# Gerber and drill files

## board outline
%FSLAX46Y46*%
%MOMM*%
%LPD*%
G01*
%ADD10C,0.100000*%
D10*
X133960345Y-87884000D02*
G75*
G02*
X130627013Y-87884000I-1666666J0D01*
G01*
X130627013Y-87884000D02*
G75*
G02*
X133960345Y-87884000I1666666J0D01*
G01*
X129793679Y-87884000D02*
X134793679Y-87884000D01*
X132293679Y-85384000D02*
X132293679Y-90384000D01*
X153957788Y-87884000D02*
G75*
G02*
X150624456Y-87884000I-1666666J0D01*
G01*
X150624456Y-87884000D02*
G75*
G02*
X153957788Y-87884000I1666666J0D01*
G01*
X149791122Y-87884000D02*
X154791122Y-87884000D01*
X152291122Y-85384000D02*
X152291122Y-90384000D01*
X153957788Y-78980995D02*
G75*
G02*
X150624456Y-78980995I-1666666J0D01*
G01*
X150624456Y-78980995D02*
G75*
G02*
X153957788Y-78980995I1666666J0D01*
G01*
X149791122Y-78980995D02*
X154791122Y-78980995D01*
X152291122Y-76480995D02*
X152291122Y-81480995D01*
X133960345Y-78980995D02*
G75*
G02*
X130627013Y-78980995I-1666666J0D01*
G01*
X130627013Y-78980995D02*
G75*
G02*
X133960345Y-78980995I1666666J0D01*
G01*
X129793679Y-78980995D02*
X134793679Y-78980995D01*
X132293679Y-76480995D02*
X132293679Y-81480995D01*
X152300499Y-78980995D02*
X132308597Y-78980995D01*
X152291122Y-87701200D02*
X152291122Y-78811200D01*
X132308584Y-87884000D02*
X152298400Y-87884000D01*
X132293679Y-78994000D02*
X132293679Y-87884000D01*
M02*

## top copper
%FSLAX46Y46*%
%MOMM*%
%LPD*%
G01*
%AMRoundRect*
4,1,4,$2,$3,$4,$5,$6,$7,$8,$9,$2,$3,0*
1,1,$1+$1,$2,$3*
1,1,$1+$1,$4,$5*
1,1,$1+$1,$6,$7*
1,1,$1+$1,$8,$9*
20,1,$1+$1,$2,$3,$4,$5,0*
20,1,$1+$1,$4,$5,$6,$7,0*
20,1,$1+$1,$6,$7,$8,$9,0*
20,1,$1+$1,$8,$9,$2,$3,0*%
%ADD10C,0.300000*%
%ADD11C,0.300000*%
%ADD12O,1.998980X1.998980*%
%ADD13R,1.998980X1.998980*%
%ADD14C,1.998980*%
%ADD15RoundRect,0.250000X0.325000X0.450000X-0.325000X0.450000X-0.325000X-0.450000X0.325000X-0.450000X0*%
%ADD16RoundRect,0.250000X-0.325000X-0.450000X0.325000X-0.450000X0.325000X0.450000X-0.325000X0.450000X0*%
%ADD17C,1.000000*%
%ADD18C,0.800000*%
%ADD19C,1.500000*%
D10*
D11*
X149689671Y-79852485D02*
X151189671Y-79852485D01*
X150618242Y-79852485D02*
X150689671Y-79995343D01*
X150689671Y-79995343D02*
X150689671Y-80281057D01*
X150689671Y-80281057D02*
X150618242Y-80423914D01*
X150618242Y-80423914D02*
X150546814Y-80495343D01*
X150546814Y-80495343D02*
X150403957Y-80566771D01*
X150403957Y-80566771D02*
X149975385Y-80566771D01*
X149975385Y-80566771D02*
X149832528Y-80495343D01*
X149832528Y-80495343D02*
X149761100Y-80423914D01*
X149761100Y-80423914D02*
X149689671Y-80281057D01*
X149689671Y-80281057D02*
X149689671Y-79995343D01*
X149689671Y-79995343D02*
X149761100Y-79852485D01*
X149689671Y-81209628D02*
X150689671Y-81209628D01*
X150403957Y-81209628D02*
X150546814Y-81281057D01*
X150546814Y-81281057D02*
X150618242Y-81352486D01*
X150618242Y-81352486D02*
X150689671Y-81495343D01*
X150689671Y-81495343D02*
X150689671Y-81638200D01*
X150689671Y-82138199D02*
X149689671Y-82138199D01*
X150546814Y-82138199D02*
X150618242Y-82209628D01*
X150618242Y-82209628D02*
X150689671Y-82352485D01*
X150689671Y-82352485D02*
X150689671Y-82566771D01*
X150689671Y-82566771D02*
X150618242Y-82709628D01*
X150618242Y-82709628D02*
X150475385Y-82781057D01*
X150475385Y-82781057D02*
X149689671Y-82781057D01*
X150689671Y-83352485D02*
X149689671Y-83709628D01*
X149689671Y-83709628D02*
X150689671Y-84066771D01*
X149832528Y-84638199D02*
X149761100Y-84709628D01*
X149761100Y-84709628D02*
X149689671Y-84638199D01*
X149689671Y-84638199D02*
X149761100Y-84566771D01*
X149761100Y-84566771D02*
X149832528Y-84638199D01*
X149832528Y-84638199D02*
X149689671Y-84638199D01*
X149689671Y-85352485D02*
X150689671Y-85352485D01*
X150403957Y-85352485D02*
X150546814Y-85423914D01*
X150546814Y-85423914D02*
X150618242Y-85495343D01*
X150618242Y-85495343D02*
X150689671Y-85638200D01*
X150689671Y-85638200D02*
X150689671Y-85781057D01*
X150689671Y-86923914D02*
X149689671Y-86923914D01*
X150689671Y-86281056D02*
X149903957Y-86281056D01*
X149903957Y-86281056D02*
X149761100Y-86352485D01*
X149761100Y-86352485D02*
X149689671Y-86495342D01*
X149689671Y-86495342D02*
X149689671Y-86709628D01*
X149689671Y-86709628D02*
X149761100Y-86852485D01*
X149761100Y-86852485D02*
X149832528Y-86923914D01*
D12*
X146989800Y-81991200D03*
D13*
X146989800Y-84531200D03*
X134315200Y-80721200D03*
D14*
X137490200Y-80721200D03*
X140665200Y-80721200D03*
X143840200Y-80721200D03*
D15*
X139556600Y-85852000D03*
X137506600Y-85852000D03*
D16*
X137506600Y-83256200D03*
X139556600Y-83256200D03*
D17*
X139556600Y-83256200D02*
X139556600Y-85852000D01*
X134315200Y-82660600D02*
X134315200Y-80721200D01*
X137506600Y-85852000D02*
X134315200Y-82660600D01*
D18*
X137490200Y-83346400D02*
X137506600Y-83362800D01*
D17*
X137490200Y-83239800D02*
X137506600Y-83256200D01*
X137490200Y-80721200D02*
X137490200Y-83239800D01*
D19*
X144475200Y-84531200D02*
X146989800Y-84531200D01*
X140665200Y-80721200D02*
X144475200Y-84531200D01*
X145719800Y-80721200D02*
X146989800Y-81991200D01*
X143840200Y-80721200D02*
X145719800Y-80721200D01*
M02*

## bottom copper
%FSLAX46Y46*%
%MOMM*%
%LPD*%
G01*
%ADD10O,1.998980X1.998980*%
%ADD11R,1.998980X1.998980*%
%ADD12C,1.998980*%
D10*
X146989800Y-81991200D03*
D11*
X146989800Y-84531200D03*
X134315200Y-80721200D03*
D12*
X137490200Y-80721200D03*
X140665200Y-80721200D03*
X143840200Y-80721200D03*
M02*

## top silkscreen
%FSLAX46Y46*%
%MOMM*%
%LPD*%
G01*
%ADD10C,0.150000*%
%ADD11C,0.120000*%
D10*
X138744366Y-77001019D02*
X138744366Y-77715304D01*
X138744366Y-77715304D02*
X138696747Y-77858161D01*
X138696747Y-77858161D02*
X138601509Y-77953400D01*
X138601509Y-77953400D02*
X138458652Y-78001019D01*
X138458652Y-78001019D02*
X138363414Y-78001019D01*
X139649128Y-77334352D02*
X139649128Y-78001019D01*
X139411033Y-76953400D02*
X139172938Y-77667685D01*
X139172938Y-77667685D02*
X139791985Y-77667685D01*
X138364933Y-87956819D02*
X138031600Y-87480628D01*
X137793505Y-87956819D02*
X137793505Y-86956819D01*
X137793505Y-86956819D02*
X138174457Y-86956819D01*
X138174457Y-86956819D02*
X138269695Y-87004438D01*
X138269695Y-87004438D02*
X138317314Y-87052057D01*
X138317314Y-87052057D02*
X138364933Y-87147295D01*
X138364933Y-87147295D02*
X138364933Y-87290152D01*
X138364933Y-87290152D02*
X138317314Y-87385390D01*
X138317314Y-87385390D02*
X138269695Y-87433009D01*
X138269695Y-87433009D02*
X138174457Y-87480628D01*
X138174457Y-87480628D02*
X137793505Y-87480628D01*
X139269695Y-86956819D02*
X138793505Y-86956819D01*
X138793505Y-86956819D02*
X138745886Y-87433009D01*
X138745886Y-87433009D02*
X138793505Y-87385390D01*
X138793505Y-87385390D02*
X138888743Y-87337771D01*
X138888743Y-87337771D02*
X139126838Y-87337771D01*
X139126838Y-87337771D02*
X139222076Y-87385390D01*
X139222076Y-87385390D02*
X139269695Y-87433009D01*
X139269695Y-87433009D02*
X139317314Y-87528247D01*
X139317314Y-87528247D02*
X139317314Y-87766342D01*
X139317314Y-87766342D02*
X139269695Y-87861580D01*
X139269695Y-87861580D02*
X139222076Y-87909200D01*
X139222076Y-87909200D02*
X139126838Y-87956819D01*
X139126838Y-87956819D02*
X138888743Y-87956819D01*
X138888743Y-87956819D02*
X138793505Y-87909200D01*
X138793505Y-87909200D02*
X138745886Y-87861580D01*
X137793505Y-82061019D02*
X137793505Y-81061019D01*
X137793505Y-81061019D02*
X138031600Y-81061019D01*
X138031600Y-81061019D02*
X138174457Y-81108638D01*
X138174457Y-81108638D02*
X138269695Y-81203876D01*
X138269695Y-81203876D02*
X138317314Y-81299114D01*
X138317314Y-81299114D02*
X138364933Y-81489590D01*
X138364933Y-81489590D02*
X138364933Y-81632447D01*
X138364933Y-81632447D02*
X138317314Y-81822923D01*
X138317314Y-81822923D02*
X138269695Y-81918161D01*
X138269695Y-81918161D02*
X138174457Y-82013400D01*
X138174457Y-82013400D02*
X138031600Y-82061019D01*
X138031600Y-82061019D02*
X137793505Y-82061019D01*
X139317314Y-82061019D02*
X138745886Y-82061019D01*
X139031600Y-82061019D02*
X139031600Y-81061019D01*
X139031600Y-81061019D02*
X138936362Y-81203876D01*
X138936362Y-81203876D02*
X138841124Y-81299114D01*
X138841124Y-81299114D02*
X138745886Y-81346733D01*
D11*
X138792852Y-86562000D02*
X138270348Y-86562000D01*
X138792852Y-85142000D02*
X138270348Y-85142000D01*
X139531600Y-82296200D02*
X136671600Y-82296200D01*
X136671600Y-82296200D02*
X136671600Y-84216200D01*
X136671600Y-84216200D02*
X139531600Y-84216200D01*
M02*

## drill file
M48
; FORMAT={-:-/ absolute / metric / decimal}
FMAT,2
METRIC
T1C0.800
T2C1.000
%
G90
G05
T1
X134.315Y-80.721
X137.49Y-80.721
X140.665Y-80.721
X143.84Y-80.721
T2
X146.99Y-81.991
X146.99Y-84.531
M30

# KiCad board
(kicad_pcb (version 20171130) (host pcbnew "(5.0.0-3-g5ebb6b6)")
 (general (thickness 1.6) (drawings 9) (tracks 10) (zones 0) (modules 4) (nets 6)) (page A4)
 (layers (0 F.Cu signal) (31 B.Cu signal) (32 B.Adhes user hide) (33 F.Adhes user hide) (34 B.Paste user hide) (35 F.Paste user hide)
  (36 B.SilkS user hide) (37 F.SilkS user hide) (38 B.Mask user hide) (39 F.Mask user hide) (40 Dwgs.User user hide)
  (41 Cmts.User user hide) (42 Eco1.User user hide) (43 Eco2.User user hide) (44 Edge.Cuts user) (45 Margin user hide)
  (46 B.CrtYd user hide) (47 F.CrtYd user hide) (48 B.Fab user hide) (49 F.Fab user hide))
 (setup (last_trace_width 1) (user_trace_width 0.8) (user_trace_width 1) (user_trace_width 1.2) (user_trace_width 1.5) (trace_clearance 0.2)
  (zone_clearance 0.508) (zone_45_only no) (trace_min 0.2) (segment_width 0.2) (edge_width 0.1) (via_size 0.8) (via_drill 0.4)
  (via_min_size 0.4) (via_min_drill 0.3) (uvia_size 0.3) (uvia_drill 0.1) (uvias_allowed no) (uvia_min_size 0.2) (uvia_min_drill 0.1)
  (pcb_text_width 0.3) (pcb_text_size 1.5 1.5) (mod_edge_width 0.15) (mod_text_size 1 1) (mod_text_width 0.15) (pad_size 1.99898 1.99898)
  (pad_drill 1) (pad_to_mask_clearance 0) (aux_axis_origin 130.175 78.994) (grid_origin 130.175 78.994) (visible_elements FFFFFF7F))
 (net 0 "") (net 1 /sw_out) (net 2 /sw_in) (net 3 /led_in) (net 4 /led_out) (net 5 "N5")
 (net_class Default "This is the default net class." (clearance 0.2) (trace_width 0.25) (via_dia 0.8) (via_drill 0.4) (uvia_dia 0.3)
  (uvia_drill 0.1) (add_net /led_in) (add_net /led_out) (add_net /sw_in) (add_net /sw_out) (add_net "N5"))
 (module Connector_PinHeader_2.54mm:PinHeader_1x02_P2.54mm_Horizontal (layer B.Cu) (at 146.9898 84.5312)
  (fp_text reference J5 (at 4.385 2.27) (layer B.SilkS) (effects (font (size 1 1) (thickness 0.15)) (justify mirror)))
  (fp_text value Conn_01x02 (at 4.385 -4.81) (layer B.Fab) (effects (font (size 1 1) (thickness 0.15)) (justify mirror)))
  (pad 2 thru_hole oval (at 0 -2.54) (size 1.99898 1.99898) (drill 1) (layers *.Mask F.Cu) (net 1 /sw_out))
  (pad 1 thru_hole rect (at 0 0) (size 1.99898 1.99898) (drill 1) (layers *.Mask F.Cu) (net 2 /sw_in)))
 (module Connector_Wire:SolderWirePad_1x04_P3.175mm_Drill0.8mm (layer F.Cu) (at 134.3152 80.7212)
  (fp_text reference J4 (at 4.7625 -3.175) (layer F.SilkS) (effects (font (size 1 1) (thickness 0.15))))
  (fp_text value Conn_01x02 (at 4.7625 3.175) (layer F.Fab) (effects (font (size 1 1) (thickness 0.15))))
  (pad 1 thru_hole rect (at 0 0) (size 1.99898 1.99898) (drill 0.8001) (layers *.Cu *.Mask) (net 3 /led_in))
  (pad 2 thru_hole circle (at 3.175 0) (size 1.99898 1.99898) (drill 0.8001) (layers *.Cu *.Mask) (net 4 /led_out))
  (pad 3 thru_hole circle (at 6.35 0) (size 1.99898 1.99898) (drill 0.8001) (layers *.Cu *.Mask) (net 2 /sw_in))
  (pad 4 thru_hole circle (at 9.525 0) (size 1.99898 1.99898) (drill 0.8001) (layers *.Cu *.Mask) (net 1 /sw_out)))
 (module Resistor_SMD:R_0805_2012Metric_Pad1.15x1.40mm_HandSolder (layer F.Cu) (at 138.5316 85.852 180)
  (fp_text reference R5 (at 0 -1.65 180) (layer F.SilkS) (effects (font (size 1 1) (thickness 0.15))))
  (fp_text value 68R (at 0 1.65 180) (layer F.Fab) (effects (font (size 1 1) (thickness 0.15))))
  (fp_line (start -0.261252 -0.71) (end 0.261252 -0.71) (layer F.SilkS) (width 0.12))
  (fp_line (start -0.261252 0.71) (end 0.261252 0.71) (layer F.SilkS) (width 0.12))
  (pad 1 smd roundrect (at -1.025 0 180) (size 1.15 1.4) (layers F.Cu F.Paste F.Mask) (roundrect_rratio 0.217391) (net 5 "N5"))
  (pad 2 smd roundrect (at 1.025 0 180) (size 1.15 1.4) (layers F.Cu F.Paste F.Mask) (roundrect_rratio 0.217391) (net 3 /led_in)))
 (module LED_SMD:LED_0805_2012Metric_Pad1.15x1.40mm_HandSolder (layer F.Cu) (at 138.5316 83.2562)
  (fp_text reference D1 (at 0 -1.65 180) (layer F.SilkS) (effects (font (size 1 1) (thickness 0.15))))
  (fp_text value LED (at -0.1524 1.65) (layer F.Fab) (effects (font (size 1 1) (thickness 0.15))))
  (fp_line (start 1 -0.96) (end -1.86 -0.96) (layer F.SilkS) (width 0.12))
  (fp_line (start -1.86 -0.96) (end -1.86 0.96) (layer F.SilkS) (width 0.12))
  (fp_line (start -1.86 0.96) (end 1 0.96) (layer F.SilkS) (width 0.12))
  (pad 1 smd roundrect (at -1.025 0) (size 1.15 1.4) (layers F.Cu F.Paste F.Mask) (roundrect_rratio 0.217391) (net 4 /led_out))
  (pad 2 smd roundrect (at 1.025 0) (size 1.15 1.4) (layers F.Cu F.Paste F.Mask) (roundrect_rratio 0.217391) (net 5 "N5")))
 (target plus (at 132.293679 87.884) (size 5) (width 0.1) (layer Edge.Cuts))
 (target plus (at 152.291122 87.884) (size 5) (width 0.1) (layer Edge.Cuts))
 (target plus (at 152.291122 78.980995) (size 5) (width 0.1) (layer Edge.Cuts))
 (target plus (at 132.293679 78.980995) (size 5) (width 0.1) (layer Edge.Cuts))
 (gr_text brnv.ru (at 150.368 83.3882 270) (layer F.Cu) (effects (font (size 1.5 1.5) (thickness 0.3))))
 (gr_line (start 152.300499 78.980995) (end 132.308597 78.980995) (layer Edge.Cuts) (width 0.1))
 (gr_line (start 152.291122 87.7012) (end 152.291122 78.8112) (layer Edge.Cuts) (width 0.1))
 (gr_line (start 132.308584 87.884) (end 152.2984 87.884) (layer Edge.Cuts) (width 0.1))
 (gr_line (start 132.293679 78.994) (end 132.293679 87.884) (layer Edge.Cuts) (width 0.1))
 (segment (start 139.5566 83.2562) (end 139.5566 85.852) (width 1) (layer F.Cu) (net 5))
 (segment (start 134.3152 82.6606) (end 134.3152 80.7212) (width 1) (layer F.Cu) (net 3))
 (segment (start 137.5066 85.852) (end 134.3152 82.6606) (width 1) (layer F.Cu) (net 3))
 (segment (start 137.4902 83.3464) (end 137.5066 83.3628) (width 0.8) (layer F.Cu) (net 4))
 (segment (start 137.4902 83.2398) (end 137.5066 83.2562) (width 1) (layer F.Cu) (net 4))
 (segment (start 137.4902 80.7212) (end 137.4902 83.2398) (width 1) (layer F.Cu) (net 4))
 (segment (start 144.4752 84.5312) (end 146.9898 84.5312) (width 1.5) (layer F.Cu) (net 2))
 (segment (start 140.6652 80.7212) (end 144.4752 84.5312) (width 1.5) (layer F.Cu) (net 2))
 (segment (start 145.7198 80.7212) (end 146.9898 81.9912) (width 1.5) (layer F.Cu) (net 1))
 (segment (start 143.8402 80.7212) (end 145.7198 80.7212) (width 1.5) (layer F.Cu) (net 1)))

